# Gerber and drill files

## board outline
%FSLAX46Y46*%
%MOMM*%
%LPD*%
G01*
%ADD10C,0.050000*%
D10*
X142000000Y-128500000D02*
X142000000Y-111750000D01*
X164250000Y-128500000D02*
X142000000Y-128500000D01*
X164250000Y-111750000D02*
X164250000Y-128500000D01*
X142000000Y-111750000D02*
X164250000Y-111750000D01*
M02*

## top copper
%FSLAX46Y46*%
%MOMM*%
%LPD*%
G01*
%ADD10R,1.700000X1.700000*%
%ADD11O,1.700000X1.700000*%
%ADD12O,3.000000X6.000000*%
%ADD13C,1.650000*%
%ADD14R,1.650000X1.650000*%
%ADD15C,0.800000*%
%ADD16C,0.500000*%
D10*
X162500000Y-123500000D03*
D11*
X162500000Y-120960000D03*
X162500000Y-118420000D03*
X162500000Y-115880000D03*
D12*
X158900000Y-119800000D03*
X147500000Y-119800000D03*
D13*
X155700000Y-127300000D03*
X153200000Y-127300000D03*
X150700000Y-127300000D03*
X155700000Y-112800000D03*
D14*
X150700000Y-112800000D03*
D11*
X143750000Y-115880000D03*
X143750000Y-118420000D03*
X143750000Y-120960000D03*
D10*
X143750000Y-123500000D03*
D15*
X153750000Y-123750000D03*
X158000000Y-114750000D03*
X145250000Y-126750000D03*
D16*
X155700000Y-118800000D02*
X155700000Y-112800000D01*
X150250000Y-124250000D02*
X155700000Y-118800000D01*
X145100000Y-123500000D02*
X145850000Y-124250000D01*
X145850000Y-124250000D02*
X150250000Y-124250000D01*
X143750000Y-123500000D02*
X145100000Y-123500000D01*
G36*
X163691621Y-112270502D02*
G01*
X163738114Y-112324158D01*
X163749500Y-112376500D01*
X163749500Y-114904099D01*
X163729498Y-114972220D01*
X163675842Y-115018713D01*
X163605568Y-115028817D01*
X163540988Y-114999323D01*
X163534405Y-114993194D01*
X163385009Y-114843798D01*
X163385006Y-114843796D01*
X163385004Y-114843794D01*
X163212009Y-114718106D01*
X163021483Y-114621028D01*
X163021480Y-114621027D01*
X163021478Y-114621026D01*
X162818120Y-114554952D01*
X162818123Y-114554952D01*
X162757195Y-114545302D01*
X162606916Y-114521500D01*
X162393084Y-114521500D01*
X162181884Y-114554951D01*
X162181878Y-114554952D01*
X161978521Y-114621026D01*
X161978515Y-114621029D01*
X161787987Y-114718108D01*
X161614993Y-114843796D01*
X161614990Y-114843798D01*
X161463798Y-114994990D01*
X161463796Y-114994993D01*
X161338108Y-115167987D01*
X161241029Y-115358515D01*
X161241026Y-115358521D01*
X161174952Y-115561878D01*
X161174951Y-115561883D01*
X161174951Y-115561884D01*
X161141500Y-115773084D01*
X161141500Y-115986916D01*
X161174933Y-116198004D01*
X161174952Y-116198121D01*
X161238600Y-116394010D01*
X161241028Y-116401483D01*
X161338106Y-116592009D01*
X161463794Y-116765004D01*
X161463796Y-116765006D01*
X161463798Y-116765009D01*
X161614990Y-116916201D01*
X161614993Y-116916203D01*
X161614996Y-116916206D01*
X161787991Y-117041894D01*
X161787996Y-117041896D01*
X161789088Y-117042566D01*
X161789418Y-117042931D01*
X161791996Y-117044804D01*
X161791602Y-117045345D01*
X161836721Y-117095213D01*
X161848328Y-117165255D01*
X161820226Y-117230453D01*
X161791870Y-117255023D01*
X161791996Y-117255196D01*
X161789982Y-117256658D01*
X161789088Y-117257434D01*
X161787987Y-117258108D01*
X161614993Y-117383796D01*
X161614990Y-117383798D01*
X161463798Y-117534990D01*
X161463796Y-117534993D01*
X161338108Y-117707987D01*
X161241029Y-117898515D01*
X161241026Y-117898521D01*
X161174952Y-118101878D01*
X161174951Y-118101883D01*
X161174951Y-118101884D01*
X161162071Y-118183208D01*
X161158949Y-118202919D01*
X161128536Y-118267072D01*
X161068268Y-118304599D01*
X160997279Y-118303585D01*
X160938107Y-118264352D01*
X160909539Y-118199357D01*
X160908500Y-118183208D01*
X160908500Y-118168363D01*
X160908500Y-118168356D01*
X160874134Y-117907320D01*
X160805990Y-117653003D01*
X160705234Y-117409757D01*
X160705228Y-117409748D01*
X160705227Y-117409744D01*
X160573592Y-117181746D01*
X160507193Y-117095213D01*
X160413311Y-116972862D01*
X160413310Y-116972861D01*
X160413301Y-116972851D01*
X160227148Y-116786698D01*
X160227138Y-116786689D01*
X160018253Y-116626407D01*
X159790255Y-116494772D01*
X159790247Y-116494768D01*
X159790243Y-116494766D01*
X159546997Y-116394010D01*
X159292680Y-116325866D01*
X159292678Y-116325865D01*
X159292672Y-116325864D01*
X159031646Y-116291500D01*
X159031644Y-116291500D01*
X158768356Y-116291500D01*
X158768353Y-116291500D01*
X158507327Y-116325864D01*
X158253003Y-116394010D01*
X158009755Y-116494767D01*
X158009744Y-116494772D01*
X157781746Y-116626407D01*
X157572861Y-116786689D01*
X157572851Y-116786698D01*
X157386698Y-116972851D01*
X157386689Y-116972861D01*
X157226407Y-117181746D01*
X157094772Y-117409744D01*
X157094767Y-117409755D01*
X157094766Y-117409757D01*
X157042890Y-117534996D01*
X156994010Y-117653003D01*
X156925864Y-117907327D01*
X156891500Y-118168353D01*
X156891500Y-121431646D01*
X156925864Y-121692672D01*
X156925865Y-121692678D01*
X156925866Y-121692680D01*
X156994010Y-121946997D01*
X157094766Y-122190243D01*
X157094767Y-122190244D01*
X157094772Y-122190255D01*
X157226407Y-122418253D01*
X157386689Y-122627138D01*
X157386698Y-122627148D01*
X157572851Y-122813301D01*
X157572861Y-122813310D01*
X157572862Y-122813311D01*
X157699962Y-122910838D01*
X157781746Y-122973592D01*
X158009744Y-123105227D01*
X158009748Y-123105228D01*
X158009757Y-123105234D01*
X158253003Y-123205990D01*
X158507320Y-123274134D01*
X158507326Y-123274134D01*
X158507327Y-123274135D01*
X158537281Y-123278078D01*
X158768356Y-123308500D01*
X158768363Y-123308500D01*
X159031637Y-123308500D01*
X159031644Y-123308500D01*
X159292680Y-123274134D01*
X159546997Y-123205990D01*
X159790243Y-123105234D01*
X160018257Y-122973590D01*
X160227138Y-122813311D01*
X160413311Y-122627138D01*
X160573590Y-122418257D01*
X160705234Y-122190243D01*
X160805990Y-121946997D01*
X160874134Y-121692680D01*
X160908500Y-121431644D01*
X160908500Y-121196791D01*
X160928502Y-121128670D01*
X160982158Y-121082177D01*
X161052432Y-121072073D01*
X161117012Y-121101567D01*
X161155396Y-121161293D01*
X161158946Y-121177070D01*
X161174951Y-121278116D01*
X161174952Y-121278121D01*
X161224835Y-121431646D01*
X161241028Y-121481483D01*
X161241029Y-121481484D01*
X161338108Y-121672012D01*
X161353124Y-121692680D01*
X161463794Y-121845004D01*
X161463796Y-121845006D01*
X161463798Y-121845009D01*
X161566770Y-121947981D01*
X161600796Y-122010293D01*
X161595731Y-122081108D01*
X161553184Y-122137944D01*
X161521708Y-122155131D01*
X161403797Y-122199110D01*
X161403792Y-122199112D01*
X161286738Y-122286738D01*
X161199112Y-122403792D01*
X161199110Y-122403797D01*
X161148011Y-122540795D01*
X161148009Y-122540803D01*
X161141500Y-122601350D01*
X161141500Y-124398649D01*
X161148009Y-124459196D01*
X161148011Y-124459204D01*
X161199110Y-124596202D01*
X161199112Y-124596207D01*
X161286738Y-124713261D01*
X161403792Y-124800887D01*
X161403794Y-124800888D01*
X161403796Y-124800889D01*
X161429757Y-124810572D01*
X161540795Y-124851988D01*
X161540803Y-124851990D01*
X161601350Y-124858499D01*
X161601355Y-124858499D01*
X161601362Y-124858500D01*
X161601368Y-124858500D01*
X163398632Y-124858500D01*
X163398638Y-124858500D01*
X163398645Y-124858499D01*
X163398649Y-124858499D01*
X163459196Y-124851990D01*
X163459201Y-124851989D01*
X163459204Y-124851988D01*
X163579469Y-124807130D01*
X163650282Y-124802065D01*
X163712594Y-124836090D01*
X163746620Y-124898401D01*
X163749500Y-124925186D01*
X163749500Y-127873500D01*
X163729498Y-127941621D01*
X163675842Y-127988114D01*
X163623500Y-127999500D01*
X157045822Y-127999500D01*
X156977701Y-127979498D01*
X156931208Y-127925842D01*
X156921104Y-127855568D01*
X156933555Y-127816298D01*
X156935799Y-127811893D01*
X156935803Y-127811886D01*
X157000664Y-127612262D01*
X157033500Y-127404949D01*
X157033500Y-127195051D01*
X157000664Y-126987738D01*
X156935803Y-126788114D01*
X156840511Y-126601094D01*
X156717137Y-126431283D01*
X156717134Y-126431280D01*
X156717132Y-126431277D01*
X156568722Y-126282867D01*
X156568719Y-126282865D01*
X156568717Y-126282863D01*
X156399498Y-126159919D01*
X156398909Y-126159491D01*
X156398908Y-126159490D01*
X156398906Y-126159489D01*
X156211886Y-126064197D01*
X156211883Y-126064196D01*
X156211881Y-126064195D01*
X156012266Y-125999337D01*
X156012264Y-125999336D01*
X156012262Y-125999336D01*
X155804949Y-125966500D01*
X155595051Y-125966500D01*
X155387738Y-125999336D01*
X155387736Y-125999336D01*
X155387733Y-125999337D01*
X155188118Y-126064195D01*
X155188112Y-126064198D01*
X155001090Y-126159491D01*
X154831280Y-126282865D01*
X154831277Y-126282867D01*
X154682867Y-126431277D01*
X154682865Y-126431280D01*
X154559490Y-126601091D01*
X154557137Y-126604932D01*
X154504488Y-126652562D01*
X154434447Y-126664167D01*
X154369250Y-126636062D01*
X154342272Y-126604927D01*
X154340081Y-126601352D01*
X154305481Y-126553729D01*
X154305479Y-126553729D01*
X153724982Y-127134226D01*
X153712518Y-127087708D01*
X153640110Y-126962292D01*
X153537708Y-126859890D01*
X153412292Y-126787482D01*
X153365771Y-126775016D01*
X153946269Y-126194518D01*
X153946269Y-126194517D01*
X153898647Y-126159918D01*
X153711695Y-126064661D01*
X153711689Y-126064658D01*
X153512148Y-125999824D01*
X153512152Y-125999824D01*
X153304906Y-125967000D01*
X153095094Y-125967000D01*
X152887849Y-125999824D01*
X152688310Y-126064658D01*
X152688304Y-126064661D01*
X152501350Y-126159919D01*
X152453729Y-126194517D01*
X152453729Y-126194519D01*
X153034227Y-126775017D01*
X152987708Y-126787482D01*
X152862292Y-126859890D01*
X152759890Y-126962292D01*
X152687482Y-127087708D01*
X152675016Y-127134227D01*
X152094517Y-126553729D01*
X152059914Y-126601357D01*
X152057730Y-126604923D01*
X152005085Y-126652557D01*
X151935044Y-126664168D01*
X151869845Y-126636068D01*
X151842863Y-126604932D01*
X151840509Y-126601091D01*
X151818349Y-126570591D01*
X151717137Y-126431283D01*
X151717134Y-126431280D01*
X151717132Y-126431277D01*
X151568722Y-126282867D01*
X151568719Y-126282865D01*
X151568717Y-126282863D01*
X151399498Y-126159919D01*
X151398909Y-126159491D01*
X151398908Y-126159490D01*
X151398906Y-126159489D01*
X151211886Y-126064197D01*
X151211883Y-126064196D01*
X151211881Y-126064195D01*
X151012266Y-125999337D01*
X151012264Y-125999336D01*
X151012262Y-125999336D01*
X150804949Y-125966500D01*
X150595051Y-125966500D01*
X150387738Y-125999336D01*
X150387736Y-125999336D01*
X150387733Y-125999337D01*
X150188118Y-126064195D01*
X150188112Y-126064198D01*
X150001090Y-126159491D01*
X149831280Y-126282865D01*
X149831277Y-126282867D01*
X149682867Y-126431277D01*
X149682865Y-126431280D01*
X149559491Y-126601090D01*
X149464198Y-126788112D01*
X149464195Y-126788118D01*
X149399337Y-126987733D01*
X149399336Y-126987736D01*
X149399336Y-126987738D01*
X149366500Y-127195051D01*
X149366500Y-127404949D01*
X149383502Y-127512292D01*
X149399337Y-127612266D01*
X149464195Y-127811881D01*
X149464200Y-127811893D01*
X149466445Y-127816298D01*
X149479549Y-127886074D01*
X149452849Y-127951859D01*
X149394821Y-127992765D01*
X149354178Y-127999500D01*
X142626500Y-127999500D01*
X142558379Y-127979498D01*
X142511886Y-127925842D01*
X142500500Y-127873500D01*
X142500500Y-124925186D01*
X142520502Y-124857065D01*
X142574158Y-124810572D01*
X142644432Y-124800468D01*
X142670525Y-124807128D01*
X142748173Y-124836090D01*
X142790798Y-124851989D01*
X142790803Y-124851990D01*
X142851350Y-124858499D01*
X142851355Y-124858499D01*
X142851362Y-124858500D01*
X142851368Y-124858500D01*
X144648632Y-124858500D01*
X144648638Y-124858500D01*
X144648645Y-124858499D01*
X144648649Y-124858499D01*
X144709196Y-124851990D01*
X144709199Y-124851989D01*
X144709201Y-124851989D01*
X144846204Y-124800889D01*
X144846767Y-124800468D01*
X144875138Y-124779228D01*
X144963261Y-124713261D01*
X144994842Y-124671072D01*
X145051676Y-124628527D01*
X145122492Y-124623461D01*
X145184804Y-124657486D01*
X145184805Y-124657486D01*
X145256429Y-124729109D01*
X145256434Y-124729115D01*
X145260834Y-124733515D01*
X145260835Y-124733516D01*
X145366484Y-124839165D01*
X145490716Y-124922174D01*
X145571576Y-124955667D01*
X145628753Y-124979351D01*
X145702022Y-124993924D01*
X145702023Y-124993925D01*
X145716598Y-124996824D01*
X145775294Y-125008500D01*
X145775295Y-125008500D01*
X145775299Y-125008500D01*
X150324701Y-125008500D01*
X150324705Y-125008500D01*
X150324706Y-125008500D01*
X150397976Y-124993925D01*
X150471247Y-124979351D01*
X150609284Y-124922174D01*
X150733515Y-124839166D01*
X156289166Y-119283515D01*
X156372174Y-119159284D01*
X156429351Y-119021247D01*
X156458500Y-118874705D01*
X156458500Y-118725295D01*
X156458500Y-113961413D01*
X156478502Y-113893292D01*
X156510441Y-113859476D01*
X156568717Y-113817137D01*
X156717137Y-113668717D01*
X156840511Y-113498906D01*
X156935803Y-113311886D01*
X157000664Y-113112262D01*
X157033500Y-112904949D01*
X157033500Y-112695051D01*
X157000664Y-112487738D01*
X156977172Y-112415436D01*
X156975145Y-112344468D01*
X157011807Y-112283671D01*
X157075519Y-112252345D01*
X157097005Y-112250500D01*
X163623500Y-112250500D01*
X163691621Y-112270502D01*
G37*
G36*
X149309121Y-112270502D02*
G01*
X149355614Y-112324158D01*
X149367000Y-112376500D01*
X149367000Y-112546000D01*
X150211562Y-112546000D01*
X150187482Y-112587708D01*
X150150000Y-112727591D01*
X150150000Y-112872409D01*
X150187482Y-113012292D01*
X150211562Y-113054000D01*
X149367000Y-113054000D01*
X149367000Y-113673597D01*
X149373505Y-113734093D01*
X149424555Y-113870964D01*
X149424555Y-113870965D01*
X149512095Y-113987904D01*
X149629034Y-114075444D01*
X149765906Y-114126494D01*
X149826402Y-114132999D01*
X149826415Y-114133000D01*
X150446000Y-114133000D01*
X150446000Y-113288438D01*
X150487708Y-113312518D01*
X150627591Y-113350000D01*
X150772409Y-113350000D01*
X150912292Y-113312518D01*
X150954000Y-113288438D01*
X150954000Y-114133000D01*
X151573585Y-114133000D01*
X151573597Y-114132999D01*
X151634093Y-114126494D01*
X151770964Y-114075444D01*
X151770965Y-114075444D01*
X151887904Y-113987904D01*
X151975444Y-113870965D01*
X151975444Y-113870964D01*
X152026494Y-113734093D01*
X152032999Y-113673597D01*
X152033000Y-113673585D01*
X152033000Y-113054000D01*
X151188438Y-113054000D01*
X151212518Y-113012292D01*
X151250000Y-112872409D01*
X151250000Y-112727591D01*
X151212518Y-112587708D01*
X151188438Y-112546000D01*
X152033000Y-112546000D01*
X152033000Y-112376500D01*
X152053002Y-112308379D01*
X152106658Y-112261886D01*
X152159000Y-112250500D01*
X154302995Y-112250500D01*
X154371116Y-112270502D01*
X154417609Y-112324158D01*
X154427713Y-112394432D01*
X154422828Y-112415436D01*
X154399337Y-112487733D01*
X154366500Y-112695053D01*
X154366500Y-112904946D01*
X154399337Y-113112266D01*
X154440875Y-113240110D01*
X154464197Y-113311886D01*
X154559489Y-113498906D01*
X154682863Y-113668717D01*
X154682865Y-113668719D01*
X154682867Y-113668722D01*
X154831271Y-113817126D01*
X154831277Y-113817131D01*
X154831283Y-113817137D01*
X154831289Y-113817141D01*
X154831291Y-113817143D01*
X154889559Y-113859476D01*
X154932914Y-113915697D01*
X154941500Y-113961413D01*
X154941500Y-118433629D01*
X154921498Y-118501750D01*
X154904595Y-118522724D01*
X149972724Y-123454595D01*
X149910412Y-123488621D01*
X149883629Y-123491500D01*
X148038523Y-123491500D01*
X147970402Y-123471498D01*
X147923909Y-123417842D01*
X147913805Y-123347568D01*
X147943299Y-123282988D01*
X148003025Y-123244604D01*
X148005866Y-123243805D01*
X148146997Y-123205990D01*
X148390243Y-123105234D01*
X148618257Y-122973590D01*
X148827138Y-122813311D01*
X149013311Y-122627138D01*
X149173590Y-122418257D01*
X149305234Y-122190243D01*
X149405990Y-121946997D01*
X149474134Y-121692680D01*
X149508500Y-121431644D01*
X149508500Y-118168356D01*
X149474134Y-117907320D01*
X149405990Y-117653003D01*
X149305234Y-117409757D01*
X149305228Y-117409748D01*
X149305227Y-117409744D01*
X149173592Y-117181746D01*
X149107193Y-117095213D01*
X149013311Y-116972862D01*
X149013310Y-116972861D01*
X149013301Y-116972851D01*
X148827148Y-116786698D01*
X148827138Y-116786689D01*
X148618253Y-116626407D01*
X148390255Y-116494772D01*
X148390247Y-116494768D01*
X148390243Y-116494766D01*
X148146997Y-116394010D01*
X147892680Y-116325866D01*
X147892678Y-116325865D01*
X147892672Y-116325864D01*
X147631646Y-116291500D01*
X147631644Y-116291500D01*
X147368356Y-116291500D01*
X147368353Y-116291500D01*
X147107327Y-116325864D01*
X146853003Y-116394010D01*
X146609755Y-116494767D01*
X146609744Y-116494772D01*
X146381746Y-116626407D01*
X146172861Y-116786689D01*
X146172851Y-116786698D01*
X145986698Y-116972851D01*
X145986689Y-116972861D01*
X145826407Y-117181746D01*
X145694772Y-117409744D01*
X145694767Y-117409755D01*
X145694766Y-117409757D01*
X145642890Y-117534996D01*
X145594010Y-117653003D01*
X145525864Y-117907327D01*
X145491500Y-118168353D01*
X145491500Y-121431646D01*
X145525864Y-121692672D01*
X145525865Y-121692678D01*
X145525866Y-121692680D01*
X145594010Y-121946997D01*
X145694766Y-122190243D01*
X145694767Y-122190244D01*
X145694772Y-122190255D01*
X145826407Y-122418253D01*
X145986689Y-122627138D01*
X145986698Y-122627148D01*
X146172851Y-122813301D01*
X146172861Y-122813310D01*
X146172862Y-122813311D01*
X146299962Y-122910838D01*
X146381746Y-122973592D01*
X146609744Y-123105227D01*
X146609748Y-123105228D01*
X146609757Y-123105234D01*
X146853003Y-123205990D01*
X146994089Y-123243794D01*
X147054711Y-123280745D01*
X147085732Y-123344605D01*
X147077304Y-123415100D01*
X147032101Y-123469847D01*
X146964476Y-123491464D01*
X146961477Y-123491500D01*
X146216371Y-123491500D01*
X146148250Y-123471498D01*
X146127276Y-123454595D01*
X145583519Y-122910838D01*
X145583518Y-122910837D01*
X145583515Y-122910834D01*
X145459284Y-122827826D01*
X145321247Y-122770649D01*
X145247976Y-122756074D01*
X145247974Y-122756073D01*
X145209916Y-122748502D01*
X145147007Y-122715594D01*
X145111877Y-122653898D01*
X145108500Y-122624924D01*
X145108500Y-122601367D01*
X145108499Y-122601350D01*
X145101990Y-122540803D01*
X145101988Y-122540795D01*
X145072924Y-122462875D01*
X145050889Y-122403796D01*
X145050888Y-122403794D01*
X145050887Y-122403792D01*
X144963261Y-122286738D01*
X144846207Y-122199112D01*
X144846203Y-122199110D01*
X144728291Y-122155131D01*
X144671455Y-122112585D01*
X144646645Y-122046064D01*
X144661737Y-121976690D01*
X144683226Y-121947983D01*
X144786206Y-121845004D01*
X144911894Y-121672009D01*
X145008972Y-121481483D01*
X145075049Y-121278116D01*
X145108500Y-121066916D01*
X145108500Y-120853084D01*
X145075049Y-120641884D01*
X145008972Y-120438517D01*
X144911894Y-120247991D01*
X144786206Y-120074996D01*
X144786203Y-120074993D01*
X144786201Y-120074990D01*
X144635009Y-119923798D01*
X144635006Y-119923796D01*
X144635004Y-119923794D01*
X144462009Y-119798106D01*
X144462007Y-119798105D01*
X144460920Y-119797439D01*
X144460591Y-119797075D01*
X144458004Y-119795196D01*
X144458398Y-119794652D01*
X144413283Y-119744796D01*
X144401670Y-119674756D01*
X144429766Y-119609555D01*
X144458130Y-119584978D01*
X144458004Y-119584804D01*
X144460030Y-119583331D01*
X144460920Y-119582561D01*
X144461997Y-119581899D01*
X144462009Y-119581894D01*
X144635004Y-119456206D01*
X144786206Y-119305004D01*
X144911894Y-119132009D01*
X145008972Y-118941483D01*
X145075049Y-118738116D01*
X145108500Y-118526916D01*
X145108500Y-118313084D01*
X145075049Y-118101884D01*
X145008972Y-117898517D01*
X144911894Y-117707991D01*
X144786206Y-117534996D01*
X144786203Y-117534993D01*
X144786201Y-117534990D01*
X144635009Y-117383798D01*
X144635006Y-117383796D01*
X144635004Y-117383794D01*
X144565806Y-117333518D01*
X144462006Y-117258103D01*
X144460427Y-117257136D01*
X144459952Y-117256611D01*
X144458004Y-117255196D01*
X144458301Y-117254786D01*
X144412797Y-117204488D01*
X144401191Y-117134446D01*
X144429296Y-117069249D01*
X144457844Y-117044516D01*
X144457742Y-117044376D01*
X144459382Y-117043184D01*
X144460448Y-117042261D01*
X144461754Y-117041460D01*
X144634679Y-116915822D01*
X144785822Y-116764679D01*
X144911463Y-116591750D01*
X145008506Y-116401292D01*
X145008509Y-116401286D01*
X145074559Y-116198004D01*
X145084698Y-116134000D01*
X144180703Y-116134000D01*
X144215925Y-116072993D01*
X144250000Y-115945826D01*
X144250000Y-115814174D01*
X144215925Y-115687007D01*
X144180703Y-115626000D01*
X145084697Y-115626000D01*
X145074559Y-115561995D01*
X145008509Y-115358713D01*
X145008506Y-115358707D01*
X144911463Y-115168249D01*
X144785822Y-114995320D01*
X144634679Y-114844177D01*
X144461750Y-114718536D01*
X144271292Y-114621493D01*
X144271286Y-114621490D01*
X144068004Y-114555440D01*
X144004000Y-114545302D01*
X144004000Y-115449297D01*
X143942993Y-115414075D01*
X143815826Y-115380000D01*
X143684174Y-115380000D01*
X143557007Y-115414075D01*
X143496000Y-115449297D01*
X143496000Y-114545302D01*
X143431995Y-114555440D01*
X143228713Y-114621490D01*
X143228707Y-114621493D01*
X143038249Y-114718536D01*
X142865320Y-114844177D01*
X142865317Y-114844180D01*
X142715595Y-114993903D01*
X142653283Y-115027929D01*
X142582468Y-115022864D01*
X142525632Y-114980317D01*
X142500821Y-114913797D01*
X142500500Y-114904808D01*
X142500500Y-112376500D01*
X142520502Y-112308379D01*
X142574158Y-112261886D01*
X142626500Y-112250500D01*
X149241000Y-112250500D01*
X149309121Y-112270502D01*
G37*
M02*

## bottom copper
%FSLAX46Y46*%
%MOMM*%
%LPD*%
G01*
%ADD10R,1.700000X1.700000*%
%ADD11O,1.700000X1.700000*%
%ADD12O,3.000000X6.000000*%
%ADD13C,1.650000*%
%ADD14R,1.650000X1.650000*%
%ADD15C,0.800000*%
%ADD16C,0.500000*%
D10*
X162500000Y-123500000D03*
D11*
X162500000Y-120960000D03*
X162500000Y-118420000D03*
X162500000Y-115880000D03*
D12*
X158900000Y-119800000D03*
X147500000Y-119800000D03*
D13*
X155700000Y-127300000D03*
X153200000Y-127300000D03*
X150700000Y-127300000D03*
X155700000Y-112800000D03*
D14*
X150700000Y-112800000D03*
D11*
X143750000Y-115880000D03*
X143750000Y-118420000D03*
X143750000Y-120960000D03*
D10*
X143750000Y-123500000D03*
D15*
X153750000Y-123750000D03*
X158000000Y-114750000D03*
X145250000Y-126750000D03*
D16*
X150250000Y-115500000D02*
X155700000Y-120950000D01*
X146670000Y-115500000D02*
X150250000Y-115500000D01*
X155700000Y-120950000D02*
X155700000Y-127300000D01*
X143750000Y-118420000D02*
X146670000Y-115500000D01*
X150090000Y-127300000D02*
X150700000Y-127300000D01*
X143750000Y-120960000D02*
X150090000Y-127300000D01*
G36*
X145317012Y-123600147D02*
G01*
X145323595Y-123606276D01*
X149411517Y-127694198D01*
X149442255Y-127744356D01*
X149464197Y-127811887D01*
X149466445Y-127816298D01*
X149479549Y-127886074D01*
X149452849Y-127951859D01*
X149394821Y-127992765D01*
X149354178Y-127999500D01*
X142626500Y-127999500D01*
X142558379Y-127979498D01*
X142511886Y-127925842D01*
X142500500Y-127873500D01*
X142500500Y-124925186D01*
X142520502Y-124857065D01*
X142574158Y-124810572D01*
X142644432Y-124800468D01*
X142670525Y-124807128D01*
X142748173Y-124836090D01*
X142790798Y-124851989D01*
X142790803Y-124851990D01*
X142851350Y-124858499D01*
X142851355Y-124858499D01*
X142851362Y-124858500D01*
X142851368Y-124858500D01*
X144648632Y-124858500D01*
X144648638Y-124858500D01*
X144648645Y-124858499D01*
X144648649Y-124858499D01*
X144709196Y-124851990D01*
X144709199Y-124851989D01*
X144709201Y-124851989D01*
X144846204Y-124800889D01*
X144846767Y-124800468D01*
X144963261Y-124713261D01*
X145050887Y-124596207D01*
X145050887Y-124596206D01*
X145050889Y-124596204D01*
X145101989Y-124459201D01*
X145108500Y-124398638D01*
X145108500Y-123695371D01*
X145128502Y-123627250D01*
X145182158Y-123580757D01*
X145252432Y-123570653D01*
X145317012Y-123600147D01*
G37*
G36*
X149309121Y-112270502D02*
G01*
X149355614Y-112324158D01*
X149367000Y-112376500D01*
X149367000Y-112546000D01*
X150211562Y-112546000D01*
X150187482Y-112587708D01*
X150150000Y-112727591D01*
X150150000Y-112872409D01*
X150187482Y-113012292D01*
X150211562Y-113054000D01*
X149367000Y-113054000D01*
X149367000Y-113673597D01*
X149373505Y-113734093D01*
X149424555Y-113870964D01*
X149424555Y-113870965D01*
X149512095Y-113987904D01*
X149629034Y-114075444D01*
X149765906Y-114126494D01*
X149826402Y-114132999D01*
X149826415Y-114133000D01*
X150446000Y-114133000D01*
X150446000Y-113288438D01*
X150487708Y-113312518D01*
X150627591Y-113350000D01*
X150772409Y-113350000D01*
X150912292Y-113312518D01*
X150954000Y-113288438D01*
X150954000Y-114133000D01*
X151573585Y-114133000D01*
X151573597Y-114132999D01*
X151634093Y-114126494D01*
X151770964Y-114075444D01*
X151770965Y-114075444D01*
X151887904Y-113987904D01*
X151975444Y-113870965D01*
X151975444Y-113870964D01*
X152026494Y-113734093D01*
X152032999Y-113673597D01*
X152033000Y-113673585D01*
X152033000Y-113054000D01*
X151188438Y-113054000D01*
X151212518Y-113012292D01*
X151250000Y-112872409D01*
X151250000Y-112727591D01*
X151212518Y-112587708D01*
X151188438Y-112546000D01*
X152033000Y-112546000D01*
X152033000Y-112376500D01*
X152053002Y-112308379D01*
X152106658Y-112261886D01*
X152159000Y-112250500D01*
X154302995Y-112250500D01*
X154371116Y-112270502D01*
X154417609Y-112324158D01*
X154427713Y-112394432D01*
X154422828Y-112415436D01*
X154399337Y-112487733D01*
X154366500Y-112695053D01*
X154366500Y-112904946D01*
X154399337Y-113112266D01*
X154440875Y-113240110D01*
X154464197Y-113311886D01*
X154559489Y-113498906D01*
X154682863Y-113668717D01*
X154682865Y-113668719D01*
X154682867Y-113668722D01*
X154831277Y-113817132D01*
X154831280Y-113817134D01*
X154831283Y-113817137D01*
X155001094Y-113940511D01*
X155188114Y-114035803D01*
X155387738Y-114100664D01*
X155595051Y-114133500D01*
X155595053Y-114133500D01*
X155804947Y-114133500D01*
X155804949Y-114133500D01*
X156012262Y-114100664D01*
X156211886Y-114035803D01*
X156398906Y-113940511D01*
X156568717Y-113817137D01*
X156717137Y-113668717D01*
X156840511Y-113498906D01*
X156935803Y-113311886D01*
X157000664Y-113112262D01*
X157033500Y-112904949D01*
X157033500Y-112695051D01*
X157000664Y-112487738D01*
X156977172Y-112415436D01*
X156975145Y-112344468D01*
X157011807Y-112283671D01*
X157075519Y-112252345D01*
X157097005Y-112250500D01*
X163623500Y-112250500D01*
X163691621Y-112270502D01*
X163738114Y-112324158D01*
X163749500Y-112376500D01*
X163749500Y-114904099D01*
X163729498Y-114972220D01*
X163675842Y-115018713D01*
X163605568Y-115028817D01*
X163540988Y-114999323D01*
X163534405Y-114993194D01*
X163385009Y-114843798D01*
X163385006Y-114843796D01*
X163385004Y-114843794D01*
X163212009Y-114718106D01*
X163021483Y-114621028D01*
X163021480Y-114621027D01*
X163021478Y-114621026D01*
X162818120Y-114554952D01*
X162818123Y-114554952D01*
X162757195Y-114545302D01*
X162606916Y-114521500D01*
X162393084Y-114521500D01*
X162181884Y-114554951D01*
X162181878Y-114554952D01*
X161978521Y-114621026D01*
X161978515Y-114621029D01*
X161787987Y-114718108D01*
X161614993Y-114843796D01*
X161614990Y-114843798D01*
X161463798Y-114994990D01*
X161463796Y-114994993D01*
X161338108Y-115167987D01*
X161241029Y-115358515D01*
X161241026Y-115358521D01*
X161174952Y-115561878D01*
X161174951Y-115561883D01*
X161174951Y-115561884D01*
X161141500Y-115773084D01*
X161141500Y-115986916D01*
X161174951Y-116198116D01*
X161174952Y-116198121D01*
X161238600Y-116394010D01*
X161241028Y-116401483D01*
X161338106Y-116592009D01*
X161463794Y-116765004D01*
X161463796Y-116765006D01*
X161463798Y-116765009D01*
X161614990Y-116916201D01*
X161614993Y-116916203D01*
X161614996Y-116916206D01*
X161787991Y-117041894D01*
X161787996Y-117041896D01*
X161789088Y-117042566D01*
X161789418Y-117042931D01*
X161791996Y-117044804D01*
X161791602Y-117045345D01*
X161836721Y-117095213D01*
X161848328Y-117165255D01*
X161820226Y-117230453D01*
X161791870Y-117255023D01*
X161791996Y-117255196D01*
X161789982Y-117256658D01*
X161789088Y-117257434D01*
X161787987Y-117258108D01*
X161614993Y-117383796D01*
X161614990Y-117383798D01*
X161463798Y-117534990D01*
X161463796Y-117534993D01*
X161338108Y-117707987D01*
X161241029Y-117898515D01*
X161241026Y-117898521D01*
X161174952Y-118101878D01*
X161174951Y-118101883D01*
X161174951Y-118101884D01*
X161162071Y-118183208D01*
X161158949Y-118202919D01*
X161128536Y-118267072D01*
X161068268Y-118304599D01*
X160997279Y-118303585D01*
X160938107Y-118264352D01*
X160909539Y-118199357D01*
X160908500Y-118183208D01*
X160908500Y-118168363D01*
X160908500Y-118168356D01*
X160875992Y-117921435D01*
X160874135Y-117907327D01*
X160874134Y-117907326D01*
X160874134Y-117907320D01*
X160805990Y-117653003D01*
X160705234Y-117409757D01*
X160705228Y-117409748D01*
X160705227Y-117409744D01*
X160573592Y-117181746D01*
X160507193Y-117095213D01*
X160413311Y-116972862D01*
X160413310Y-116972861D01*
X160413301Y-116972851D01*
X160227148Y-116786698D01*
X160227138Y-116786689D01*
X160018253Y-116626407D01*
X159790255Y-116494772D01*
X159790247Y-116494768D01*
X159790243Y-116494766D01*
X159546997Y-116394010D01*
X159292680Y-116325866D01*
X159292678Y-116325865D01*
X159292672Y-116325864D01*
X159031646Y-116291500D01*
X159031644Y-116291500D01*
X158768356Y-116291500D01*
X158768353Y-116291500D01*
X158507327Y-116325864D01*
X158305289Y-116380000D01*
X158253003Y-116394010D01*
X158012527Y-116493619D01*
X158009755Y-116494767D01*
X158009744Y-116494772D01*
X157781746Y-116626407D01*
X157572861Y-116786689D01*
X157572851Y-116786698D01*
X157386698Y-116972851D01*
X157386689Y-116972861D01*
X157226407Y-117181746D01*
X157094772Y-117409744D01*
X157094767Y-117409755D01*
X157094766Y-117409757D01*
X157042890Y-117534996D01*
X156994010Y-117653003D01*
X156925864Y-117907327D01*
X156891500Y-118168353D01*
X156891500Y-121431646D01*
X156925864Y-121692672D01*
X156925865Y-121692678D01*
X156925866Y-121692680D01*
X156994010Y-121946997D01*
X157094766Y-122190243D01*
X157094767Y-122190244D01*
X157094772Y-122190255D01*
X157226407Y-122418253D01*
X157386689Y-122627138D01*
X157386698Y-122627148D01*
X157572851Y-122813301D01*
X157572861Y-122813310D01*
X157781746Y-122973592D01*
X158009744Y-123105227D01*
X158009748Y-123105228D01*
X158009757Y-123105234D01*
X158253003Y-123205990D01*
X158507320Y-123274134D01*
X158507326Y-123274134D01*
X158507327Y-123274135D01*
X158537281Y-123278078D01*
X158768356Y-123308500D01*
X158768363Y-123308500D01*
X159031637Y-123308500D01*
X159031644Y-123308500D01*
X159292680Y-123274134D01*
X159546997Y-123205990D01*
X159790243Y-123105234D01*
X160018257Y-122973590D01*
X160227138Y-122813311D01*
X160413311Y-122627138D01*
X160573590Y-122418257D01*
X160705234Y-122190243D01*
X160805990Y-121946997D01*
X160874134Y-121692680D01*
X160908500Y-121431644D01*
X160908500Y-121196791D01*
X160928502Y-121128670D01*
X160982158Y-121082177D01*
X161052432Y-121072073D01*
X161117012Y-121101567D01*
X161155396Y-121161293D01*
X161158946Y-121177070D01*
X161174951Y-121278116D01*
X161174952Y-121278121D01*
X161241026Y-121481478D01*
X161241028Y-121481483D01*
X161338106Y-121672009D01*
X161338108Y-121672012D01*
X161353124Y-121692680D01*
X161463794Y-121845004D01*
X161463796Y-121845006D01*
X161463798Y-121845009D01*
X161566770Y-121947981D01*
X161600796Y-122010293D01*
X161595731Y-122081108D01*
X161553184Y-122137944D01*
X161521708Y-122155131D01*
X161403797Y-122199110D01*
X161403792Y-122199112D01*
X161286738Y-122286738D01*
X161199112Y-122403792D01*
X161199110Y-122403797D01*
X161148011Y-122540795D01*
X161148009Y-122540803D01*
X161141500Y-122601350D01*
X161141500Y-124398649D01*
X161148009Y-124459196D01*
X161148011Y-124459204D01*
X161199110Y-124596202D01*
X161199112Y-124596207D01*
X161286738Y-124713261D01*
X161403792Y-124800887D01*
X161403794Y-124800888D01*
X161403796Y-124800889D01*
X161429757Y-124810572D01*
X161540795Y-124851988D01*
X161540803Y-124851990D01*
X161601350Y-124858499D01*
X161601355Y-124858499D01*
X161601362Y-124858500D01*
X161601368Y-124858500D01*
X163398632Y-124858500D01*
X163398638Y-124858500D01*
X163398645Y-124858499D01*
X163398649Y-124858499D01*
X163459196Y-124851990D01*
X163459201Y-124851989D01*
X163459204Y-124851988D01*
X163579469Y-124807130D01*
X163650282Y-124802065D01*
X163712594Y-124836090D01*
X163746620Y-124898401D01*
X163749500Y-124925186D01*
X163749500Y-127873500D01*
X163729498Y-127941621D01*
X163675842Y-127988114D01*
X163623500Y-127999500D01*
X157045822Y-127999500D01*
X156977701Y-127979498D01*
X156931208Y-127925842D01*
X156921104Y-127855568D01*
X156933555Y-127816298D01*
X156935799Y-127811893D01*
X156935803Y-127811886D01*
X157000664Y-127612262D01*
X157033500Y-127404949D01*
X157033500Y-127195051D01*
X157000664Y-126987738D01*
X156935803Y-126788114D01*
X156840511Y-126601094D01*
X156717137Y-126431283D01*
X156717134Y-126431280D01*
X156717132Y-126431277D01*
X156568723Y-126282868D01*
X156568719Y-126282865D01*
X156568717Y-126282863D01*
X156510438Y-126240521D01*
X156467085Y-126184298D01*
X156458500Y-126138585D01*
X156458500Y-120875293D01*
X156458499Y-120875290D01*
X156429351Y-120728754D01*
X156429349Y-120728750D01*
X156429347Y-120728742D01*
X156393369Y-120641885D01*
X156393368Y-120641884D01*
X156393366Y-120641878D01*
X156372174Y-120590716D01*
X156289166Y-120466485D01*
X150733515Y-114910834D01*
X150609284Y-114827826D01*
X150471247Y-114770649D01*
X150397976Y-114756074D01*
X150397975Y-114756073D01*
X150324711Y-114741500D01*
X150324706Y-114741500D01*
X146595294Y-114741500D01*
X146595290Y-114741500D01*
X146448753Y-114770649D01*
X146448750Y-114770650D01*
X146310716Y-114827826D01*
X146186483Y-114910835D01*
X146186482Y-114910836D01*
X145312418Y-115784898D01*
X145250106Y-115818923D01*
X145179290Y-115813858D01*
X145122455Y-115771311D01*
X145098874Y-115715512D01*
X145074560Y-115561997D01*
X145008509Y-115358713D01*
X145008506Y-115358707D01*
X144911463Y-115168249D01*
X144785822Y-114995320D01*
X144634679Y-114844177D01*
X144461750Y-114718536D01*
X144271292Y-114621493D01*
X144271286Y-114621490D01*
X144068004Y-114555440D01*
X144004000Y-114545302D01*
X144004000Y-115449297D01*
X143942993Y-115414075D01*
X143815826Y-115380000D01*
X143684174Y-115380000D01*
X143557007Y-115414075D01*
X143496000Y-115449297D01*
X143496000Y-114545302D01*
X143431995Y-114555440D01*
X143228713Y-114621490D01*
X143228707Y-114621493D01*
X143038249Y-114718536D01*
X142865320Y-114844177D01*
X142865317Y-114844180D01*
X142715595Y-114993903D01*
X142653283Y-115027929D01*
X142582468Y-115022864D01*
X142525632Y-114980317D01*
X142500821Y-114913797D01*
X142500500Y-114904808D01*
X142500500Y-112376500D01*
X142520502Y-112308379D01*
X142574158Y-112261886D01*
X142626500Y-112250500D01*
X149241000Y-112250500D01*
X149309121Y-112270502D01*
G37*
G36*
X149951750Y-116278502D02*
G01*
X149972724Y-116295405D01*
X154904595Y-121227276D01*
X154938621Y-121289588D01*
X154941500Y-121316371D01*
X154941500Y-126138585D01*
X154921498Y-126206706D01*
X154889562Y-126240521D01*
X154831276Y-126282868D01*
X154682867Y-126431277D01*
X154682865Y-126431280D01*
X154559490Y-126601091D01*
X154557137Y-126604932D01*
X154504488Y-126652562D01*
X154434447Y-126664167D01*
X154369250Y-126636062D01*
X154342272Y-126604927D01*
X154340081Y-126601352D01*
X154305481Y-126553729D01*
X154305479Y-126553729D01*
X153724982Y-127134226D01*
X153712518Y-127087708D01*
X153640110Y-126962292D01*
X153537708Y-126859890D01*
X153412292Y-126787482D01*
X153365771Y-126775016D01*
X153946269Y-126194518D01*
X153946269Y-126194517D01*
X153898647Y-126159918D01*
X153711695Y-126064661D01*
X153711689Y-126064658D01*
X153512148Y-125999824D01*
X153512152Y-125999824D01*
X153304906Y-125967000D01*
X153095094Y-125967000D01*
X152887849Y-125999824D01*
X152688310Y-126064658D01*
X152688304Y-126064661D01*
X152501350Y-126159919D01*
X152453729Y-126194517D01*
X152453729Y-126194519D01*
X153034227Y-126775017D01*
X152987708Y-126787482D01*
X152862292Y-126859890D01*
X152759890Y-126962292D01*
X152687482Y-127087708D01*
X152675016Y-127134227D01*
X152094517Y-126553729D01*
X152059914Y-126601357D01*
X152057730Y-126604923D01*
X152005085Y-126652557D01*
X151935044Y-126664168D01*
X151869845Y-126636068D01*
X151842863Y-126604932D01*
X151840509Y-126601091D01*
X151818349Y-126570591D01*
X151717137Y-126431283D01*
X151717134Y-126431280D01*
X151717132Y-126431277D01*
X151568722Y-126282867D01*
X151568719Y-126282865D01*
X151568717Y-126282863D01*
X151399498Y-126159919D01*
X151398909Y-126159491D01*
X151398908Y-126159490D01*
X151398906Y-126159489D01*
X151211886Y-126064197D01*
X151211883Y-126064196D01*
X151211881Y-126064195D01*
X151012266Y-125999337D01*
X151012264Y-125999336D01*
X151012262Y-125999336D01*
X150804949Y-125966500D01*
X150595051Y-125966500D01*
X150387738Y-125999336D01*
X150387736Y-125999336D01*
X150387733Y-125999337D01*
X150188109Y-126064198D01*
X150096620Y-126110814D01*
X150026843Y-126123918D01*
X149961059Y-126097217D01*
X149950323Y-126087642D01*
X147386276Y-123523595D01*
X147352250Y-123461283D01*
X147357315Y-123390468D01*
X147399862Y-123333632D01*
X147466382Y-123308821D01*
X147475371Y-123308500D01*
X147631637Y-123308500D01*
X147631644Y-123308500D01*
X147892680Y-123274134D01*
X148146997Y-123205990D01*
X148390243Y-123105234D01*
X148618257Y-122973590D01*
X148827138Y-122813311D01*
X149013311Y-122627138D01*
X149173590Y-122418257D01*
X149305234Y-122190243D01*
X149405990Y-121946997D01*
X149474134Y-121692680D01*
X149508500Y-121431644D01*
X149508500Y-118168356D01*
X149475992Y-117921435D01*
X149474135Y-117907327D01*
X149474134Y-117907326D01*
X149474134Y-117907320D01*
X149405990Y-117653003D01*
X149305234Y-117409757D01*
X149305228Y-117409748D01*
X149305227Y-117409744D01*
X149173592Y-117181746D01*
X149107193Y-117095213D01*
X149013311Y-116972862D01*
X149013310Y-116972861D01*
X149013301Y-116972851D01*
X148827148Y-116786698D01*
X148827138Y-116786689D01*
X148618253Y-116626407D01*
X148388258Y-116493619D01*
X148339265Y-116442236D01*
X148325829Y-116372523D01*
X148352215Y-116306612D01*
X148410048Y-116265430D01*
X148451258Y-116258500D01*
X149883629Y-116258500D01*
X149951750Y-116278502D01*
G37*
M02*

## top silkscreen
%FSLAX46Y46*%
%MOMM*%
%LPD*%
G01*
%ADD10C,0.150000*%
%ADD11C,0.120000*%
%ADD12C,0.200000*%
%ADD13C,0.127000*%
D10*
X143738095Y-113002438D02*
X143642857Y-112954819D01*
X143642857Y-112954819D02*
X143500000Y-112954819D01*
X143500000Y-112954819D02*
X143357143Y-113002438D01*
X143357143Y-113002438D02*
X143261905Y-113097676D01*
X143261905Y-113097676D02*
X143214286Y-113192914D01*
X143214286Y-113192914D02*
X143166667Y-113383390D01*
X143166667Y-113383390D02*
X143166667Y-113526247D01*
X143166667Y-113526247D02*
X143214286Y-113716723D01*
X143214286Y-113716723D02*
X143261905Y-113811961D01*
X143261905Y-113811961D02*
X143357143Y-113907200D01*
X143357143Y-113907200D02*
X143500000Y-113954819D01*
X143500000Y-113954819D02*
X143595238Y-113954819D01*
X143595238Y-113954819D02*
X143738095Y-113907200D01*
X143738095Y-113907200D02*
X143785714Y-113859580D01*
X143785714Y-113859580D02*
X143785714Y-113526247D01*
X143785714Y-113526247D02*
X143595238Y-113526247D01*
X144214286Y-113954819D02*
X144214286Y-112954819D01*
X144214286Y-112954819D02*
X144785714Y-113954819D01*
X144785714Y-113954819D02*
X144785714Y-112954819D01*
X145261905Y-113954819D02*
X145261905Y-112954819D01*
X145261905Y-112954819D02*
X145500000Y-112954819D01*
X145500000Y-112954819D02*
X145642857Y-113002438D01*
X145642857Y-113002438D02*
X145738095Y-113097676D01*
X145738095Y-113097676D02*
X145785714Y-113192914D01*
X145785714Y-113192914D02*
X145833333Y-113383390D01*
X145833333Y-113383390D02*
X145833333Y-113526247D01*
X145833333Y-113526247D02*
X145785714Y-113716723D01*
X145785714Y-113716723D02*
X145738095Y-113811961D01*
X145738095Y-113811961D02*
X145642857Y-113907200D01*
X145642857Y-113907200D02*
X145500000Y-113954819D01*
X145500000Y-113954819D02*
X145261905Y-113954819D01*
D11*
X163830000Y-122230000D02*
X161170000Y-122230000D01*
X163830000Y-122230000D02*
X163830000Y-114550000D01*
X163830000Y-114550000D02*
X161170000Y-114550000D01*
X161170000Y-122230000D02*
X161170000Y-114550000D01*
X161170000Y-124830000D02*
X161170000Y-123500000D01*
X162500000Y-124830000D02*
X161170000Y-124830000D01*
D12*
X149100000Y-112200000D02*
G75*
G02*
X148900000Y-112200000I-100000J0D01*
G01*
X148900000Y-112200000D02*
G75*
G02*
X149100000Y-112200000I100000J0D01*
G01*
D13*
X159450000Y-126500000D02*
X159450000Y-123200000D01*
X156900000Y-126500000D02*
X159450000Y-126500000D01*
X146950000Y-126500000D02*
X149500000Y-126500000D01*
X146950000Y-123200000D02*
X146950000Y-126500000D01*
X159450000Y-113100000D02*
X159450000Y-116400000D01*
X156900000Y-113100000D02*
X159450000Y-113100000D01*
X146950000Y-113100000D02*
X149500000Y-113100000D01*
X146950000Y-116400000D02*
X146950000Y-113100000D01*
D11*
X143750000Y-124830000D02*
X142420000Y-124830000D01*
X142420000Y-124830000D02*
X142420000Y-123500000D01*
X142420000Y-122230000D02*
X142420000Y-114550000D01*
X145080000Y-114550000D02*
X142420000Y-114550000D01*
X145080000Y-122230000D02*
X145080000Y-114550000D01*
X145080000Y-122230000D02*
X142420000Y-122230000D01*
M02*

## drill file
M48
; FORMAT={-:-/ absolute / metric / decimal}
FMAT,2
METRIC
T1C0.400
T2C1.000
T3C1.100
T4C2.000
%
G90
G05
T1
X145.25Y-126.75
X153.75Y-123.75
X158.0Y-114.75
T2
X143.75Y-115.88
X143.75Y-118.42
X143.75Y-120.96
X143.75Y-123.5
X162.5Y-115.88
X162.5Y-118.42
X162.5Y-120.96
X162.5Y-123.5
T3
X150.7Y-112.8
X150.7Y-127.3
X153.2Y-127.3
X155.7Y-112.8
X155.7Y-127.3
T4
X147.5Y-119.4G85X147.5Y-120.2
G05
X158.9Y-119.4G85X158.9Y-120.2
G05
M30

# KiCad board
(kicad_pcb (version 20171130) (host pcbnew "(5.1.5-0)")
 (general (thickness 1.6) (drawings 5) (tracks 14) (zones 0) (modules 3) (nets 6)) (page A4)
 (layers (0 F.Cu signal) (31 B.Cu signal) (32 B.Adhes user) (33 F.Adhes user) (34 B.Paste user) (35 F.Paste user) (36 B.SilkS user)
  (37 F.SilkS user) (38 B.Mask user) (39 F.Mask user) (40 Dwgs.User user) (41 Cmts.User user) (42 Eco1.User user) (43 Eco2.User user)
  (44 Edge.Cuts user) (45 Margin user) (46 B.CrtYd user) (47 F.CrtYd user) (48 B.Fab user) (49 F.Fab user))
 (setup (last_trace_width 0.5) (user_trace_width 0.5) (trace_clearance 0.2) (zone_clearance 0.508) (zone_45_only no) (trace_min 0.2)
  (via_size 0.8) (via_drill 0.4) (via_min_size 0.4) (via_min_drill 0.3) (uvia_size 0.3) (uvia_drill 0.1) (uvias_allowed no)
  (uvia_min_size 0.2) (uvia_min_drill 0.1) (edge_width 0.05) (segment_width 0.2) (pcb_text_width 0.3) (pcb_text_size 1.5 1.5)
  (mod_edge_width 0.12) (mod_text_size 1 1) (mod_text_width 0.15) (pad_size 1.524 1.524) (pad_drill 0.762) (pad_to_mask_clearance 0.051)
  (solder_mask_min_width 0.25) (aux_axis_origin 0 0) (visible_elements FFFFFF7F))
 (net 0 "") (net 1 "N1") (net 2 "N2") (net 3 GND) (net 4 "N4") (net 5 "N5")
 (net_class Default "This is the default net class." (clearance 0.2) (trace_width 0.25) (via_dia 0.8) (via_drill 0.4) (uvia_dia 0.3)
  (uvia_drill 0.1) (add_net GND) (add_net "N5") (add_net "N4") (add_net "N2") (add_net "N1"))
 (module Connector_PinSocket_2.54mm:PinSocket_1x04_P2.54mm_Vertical (layer F.Cu) (at 162.5 123.5 180)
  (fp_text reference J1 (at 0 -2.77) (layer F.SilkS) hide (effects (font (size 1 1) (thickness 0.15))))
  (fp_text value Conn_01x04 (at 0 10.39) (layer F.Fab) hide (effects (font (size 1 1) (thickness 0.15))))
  (fp_line (start -1.33 1.27) (end 1.33 1.27) (layer F.SilkS) (width 0.12))
  (fp_line (start -1.33 1.27) (end -1.33 8.95) (layer F.SilkS) (width 0.12))
  (fp_line (start -1.33 8.95) (end 1.33 8.95) (layer F.SilkS) (width 0.12))
  (fp_line (start 1.33 1.27) (end 1.33 8.95) (layer F.SilkS) (width 0.12))
  (fp_line (start 1.33 -1.33) (end 1.33 0) (layer F.SilkS) (width 0.12))
  (fp_line (start 0 -1.33) (end 1.33 -1.33) (layer F.SilkS) (width 0.12))
  (pad 1 thru_hole rect (at 0 0 180) (size 1.7 1.7) (drill 1) (layers *.Cu *.Mask))
  (pad 2 thru_hole oval (at 0 2.54 180) (size 1.7 1.7) (drill 1) (layers *.Cu *.Mask))
  (pad 3 thru_hole oval (at 0 5.08 180) (size 1.7 1.7) (drill 1) (layers *.Cu *.Mask))
  (pad 4 thru_hole oval (at 0 7.62 180) (size 1.7 1.7) (drill 1) (layers *.Cu *.Mask)))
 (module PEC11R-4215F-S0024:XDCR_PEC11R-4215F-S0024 (layer F.Cu) (at 153.2 119.8)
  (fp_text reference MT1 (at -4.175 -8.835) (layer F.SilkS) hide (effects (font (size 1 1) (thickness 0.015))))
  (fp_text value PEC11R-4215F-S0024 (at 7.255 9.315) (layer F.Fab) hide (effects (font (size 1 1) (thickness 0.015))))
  (fp_circle (center -4.2 -7.6) (end -4.1 -7.6) (layer F.SilkS) (width 0.2))
  (fp_line (start 6.25 6.7) (end 6.25 3.4) (layer F.SilkS) (width 0.127))
  (fp_line (start 3.7 6.7) (end 6.25 6.7) (layer F.SilkS) (width 0.127))
  (fp_line (start -6.25 6.7) (end -3.7 6.7) (layer F.SilkS) (width 0.127))
  (fp_line (start -6.25 3.4) (end -6.25 6.7) (layer F.SilkS) (width 0.127))
  (fp_line (start 6.25 -6.7) (end 6.25 -3.4) (layer F.SilkS) (width 0.127))
  (fp_line (start 3.7 -6.7) (end 6.25 -6.7) (layer F.SilkS) (width 0.127))
  (fp_line (start -6.25 -6.7) (end -3.7 -6.7) (layer F.SilkS) (width 0.127))
  (fp_line (start -6.25 -3.4) (end -6.25 -6.7) (layer F.SilkS) (width 0.127))
  (pad S2 thru_hole oval (at 5.7 0) (size 3 6) (drill oval 2 2.8) (layers *.Cu *.Mask) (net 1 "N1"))
  (pad S1 thru_hole oval (at -5.7 0) (size 3 6) (drill oval 2 2.8) (layers *.Cu *.Mask) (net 1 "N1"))
  (pad B thru_hole circle (at 2.5 7.5) (size 1.65 1.65) (drill 1.1) (layers *.Cu *.Mask) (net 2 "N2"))
  (pad COM thru_hole circle (at 0 7.5) (size 1.65 1.65) (drill 1.1) (layers *.Cu *.Mask) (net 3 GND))
  (pad A thru_hole circle (at -2.5 7.5) (size 1.65 1.65) (drill 1.1) (layers *.Cu *.Mask) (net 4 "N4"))
  (pad 2 thru_hole circle (at 2.5 -7) (size 1.65 1.65) (drill 1.1) (layers *.Cu *.Mask) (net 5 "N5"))
  (pad 1 thru_hole rect (at -2.5 -7) (size 1.65 1.65) (drill 1.1) (layers *.Cu *.Mask) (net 3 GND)))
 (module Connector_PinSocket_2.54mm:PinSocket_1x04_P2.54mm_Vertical (layer F.Cu) (at 143.75 123.5 180)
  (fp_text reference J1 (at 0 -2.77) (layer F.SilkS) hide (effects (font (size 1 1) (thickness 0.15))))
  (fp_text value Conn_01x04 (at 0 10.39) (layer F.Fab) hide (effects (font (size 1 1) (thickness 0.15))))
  (fp_line (start 0 -1.33) (end 1.33 -1.33) (layer F.SilkS) (width 0.12))
  (fp_line (start 1.33 -1.33) (end 1.33 0) (layer F.SilkS) (width 0.12))
  (fp_line (start 1.33 1.27) (end 1.33 8.95) (layer F.SilkS) (width 0.12))
  (fp_line (start -1.33 8.95) (end 1.33 8.95) (layer F.SilkS) (width 0.12))
  (fp_line (start -1.33 1.27) (end -1.33 8.95) (layer F.SilkS) (width 0.12))
  (fp_line (start -1.33 1.27) (end 1.33 1.27) (layer F.SilkS) (width 0.12))
  (pad 4 thru_hole oval (at 0 7.62 180) (size 1.7 1.7) (drill 1) (layers *.Cu *.Mask) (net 3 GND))
  (pad 3 thru_hole oval (at 0 5.08 180) (size 1.7 1.7) (drill 1) (layers *.Cu *.Mask) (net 2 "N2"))
  (pad 2 thru_hole oval (at 0 2.54 180) (size 1.7 1.7) (drill 1) (layers *.Cu *.Mask) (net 4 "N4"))
  (pad 1 thru_hole rect (at 0 0 180) (size 1.7 1.7) (drill 1) (layers *.Cu *.Mask) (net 5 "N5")))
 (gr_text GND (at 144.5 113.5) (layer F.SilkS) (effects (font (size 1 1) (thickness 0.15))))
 (gr_line (start 142 128.5) (end 142 111.75) (layer Edge.Cuts) (width 0.05))
 (gr_line (start 164.25 128.5) (end 142 128.5) (layer Edge.Cuts) (width 0.05))
 (gr_line (start 164.25 111.75) (end 164.25 128.5) (layer Edge.Cuts) (width 0.05))
 (gr_line (start 142 111.75) (end 164.25 111.75) (layer Edge.Cuts) (width 0.05))
 (via (at 153.75 123.75) (size 0.8) (drill 0.4) (layers F.Cu B.Cu) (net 3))
 (via (at 158 114.75) (size 0.8) (drill 0.4) (layers F.Cu B.Cu) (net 3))
 (via (at 145.25 126.75) (size 0.8) (drill 0.4) (layers F.Cu B.Cu) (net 3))
 (segment (start 150.25 115.5) (end 155.7 120.95) (width 0.5) (layer B.Cu) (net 2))
 (segment (start 146.67 115.5) (end 150.25 115.5) (width 0.5) (layer B.Cu) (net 2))
 (segment (start 155.7 120.95) (end 155.7 127.3) (width 0.5) (layer B.Cu) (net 2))
 (segment (start 143.75 118.42) (end 146.67 115.5) (width 0.5) (layer B.Cu) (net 2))
 (segment (start 150.09 127.3) (end 150.7 127.3) (width 0.5) (layer B.Cu) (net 4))
 (segment (start 143.75 120.96) (end 150.09 127.3) (width 0.5) (layer B.Cu) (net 4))
 (segment (start 155.7 118.8) (end 155.7 112.8) (width 0.5) (layer F.Cu) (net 5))
 (segment (start 150.25 124.25) (end 155.7 118.8) (width 0.5) (layer F.Cu) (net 5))
 (segment (start 145.1 123.5) (end 145.85 124.25) (width 0.5) (layer F.Cu) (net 5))
 (segment (start 145.85 124.25) (end 150.25 124.25) (width 0.5) (layer F.Cu) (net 5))
 (segment (start 143.75 123.5) (end 145.1 123.5) (width 0.5) (layer F.Cu) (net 5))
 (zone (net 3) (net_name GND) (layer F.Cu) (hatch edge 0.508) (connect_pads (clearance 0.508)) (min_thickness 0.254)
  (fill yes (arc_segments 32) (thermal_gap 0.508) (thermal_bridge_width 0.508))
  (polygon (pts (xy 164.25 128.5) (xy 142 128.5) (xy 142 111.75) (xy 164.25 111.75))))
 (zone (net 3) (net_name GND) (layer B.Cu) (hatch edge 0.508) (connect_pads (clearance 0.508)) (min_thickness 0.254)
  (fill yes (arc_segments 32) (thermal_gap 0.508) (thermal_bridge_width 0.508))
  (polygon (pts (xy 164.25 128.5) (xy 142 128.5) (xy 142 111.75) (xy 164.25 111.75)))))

